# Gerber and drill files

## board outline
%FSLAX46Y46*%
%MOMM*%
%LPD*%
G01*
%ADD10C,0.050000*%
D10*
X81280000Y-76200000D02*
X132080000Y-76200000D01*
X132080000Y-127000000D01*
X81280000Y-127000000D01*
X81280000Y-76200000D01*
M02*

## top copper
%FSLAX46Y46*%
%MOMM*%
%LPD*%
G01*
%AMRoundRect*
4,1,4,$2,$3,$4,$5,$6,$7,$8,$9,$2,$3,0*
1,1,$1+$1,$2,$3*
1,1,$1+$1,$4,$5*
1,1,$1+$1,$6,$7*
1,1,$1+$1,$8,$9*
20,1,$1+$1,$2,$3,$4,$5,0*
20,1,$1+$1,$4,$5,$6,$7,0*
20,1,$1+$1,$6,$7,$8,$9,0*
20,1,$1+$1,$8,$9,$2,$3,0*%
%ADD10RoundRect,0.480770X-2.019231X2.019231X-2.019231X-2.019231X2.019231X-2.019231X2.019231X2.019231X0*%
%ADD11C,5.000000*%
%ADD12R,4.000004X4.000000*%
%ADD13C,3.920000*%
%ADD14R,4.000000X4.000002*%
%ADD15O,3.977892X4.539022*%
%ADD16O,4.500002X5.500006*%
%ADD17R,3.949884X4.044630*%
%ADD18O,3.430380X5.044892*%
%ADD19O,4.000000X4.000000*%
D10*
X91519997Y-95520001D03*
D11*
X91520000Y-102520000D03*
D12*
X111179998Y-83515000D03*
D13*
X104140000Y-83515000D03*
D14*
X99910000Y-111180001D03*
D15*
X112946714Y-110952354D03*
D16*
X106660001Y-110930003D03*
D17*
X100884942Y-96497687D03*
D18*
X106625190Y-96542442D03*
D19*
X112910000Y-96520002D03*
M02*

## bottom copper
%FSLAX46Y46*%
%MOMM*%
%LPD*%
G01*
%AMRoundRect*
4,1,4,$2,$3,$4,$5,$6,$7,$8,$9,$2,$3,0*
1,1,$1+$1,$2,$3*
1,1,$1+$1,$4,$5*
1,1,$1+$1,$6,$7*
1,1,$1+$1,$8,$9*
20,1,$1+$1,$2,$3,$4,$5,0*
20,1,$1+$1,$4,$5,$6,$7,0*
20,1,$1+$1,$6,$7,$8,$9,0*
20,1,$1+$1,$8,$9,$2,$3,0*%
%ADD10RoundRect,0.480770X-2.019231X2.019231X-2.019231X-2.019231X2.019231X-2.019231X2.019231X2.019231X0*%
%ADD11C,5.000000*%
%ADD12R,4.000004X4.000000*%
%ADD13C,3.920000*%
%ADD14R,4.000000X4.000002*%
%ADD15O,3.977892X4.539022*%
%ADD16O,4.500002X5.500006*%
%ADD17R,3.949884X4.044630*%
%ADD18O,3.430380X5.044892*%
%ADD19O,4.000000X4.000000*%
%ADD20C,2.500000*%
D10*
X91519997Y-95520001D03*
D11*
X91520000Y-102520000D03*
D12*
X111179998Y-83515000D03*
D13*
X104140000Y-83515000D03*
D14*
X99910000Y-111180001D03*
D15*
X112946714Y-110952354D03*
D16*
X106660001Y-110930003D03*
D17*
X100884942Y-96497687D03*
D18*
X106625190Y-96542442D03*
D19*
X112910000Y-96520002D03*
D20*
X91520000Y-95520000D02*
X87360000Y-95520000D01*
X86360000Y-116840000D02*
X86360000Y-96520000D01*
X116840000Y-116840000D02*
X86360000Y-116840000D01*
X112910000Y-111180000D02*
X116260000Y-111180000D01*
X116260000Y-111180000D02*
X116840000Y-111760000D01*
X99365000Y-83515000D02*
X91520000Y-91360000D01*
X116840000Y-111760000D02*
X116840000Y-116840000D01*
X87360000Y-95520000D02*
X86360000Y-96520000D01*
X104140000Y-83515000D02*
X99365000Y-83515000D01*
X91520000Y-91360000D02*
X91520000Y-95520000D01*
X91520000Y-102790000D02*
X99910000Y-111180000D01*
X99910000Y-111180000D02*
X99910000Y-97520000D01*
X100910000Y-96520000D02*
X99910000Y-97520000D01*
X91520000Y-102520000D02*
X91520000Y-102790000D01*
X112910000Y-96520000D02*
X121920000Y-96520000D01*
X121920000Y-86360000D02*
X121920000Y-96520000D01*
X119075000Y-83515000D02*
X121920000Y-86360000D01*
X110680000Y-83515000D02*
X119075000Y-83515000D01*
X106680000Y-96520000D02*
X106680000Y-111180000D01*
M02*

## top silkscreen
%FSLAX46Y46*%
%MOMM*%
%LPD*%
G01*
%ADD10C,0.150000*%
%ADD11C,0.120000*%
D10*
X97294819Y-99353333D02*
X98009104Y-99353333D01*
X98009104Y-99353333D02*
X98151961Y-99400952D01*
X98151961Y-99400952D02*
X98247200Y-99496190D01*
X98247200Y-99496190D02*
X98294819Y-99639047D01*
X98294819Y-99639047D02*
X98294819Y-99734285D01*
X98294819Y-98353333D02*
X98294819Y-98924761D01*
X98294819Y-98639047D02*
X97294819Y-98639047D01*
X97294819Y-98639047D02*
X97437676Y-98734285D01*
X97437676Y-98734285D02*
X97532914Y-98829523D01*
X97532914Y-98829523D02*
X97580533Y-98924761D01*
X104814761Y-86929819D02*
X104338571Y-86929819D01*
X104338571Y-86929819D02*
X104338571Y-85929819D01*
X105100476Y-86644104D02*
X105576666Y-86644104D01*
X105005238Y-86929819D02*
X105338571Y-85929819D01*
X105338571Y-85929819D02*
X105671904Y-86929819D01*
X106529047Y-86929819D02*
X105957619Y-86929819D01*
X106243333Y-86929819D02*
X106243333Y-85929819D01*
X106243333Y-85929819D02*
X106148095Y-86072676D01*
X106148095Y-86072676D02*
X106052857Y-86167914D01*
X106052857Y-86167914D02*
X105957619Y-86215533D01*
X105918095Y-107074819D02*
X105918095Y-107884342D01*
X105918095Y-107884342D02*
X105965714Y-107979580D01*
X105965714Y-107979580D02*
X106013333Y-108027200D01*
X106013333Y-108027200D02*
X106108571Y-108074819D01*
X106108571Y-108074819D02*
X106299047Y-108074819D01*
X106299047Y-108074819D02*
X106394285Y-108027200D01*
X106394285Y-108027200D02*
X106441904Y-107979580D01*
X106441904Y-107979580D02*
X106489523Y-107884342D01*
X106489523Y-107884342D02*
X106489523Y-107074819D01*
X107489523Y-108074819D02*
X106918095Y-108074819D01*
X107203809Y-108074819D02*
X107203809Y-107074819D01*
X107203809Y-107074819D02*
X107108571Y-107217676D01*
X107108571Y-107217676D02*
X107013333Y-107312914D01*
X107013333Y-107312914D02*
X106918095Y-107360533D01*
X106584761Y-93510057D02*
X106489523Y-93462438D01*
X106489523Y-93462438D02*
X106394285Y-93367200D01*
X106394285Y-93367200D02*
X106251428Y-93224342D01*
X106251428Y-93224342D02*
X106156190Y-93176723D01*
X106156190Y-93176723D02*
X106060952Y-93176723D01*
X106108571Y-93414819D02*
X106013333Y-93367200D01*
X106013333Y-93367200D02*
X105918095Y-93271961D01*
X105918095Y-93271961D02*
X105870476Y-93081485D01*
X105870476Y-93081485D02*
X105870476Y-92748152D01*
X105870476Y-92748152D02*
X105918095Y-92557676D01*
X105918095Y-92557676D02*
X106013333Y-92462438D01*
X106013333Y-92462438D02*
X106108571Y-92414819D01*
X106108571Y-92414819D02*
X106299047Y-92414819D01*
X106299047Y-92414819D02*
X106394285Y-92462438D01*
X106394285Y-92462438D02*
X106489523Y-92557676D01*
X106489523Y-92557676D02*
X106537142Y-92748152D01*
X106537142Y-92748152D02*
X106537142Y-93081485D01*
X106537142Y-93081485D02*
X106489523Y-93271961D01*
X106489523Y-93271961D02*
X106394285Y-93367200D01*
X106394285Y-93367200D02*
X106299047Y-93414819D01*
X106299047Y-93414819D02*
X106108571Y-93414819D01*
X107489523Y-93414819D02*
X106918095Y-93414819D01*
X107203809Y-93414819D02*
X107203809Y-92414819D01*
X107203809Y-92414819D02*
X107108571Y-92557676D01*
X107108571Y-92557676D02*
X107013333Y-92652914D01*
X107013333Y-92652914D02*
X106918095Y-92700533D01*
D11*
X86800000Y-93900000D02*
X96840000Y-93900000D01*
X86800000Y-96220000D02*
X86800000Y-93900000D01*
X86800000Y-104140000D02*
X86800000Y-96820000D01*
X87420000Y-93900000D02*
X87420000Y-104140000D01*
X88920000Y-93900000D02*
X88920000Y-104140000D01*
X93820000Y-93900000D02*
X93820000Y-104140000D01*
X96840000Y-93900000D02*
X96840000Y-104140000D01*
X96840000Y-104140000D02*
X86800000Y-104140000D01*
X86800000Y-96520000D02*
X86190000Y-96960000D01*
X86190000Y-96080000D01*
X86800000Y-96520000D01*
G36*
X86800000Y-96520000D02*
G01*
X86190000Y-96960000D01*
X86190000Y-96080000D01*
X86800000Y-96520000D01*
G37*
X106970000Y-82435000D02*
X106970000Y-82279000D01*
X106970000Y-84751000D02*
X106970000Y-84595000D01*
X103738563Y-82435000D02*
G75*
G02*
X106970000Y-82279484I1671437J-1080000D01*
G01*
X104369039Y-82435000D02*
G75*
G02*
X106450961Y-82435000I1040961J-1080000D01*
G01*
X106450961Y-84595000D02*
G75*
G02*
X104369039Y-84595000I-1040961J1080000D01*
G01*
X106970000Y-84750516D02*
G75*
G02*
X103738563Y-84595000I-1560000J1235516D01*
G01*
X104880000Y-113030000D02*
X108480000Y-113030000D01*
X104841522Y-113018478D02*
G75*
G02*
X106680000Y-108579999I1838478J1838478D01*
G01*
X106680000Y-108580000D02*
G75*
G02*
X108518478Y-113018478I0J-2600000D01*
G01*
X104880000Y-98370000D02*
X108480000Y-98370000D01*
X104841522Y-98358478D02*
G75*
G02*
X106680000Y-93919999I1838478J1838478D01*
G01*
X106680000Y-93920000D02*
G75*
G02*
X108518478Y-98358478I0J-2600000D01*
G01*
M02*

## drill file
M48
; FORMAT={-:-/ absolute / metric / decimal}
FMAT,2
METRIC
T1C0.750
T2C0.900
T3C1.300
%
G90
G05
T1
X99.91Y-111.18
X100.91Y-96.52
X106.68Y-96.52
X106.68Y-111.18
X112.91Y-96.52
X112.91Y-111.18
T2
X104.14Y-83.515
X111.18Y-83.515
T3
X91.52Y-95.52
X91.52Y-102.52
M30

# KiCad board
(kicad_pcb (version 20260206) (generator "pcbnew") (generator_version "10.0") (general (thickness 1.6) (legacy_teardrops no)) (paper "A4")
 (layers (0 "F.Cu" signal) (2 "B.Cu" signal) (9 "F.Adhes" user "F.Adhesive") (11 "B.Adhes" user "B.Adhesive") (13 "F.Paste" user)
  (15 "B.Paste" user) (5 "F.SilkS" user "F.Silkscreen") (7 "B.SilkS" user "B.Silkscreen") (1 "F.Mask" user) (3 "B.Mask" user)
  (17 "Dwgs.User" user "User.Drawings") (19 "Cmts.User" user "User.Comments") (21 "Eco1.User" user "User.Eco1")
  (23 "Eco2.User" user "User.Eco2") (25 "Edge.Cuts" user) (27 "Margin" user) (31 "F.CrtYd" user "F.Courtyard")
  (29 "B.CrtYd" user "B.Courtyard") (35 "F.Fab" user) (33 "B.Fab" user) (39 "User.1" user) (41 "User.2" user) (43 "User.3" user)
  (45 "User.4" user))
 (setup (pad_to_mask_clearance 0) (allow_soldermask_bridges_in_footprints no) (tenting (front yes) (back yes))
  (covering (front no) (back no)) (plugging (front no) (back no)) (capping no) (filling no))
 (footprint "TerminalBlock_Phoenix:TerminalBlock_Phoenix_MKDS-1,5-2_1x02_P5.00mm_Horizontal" (layer "F.Cu") (at 91.52 96.52 -90)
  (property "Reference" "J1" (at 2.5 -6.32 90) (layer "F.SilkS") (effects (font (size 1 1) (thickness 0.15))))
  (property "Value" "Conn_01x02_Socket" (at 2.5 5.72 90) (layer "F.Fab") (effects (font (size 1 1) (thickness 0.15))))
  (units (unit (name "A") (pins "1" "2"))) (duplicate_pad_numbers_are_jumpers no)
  (fp_line (start -2.62 4.72) (end -2.62 -5.32) (stroke (width 0.12) (type solid)) (layer "F.SilkS"))
  (fp_line (start -0.3 4.72) (end -2.62 4.72) (stroke (width 0.12) (type solid)) (layer "F.SilkS"))
  (fp_line (start 7.62 4.72) (end 0.3 4.72) (stroke (width 0.12) (type solid)) (layer "F.SilkS"))
  (fp_line (start -2.62 4.1) (end 7.62 4.1) (stroke (width 0.12) (type solid)) (layer "F.SilkS"))
  (fp_line (start -2.62 2.6) (end 7.62 2.6) (stroke (width 0.12) (type solid)) (layer "F.SilkS"))
  (fp_line (start -2.62 -2.3) (end 7.62 -2.3) (stroke (width 0.12) (type solid)) (layer "F.SilkS"))
  (fp_line (start -2.62 -5.32) (end 7.62 -5.32) (stroke (width 0.12) (type solid)) (layer "F.SilkS"))
  (fp_line (start 7.62 -5.32) (end 7.62 4.72) (stroke (width 0.12) (type solid)) (layer "F.SilkS"))
  (fp_poly (pts (xy 0 4.72) (xy 0.44 5.33) (xy -0.44 5.33)) (stroke (width 0.12) (type solid)) (fill yes) (layer "F.SilkS"))
  (pad "1" thru_hole roundrect (at -1 0 270) (size 5.000002 5.000002) (drill 1.3 (offset 0.000001 0.000003)) (layers "*.Cu" "*.Mask")
   (remove_unused_layers no) (roundrect_rratio 0.096154) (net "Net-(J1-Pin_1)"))
  (pad "2" thru_hole circle (at 6 0 270) (size 5 5) (drill 1.3) (layers "*.Cu" "*.Mask") (remove_unused_layers no) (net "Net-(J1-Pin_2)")))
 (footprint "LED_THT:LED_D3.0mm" (layer "F.Cu") (at 106.68 83.515 180)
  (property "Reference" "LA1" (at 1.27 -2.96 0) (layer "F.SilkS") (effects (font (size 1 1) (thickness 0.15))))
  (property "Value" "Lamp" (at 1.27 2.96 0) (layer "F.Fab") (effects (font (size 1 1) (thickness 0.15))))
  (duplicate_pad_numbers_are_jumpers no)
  (fp_line (start -0.29 1.08) (end -0.29 1.236) (stroke (width 0.12) (type solid)) (layer "F.SilkS"))
  (fp_line (start -0.29 -1.236) (end -0.29 -1.08) (stroke (width 0.12) (type solid)) (layer "F.SilkS"))
  (fp_arc (start 2.941437 1.08) (mid 1.36566 1.987699) (end -0.29 1.235516) (stroke (width 0.12) (type solid)) (layer "F.SilkS"))
  (fp_arc (start 2.310961 1.08) (mid 1.27 1.5) (end 0.229039 1.08) (stroke (width 0.12) (type solid)) (layer "F.SilkS"))
  (fp_arc (start 0.229039 -1.08) (mid 1.27 -1.5) (end 2.310961 -1.08) (stroke (width 0.12) (type solid)) (layer "F.SilkS"))
  (fp_arc (start -0.29 -1.235516) (mid 1.36566 -1.987699) (end 2.941437 -1.08) (stroke (width 0.12) (type solid)) (layer "F.SilkS"))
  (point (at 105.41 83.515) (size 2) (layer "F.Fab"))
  (pad "1" thru_hole rect (at -4.5 0 180) (size 4.000004 4) (drill 0.9 (offset 0.000002 0)) (layers "*.Cu" "*.Mask")
   (remove_unused_layers no) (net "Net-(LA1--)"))
  (pad "2" thru_hole circle (at 2.54 0 180) (size 3.92 3.92) (drill 0.9) (layers "*.Cu" "*.Mask") (remove_unused_layers no)
   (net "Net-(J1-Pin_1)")))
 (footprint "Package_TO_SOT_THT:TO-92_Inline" (layer "F.Cu") (at 105.41 111.18)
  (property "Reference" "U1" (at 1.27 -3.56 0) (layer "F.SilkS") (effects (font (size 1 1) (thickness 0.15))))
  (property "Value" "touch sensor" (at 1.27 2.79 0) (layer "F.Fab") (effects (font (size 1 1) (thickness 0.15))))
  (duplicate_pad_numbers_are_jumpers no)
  (fp_line (start -0.53 1.85) (end 3.07 1.85) (stroke (width 0.12) (type solid)) (layer "F.SilkS"))
  (fp_arc (start -0.568478 1.838478) (mid -1.132087 -0.994977) (end 1.27 -2.6) (stroke (width 0.12) (type solid)) (layer "F.SilkS"))
  (fp_arc (start 1.27 -2.6) (mid 3.672087 -0.994977) (end 3.108478 1.838478) (stroke (width 0.12) (type solid)) (layer "F.SilkS"))
  (pad "1" thru_hole rect (at -5.5 0) (size 4 4.000002) (drill 0.75 (offset 0 0.000001)) (layers "*.Cu" "*.Mask") (remove_unused_layers no)
   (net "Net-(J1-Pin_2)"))
  (pad "2" thru_hole oval (at 7.5 0) (size 3.977892 4.539022) (drill 0.75 (offset 0.036714 -0.227646)) (layers "*.Cu" "*.Mask")
   (remove_unused_layers no) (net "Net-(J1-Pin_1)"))
  (pad "3" thru_hole oval (at 1.27 0) (size 4.500002 5.500006) (drill 0.75 (offset -0.019999 -0.249997)) (layers "*.Cu" "*.Mask")
   (remove_unused_layers no) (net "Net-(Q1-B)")))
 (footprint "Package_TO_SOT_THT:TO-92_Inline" (layer "F.Cu") (at 105.41 96.52)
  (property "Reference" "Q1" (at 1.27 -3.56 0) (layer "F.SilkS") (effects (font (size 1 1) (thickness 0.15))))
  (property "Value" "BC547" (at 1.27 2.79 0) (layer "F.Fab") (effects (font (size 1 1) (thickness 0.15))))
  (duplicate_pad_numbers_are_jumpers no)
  (fp_line (start -0.53 1.85) (end 3.07 1.85) (stroke (width 0.12) (type solid)) (layer "F.SilkS"))
  (fp_arc (start -0.568478 1.838478) (mid -1.132087 -0.994977) (end 1.27 -2.6) (stroke (width 0.12) (type solid)) (layer "F.SilkS"))
  (fp_arc (start 1.27 -2.6) (mid 3.672087 -0.994977) (end 3.108478 1.838478) (stroke (width 0.12) (type solid)) (layer "F.SilkS"))
  (pad "1" thru_hole rect (at -4.5 0) (size 3.949884 4.04463) (drill 0.75 (offset -0.025058 -0.022313)) (layers "*.Cu" "*.Mask")
   (remove_unused_layers no) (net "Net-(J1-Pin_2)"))
  (pad "2" thru_hole oval (at 1.27 0) (size 3.43038 5.044892) (drill 0.75 (offset -0.05481 0.022442)) (layers "*.Cu" "*.Mask")
   (remove_unused_layers no) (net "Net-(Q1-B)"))
  (pad "3" thru_hole oval (at 7.5 0) (size 4 4) (drill 0.75 (offset 0 0.000002)) (layers "*.Cu" "*.Mask") (remove_unused_layers no)
   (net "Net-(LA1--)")))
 (gr_rect (start 81.28 76.2) (end 132.08 127) (stroke (width 0.05) (type default)) (fill no) (layer "Edge.Cuts"))
 (segment (start 91.52 95.52) (end 87.36 95.52) (width 2.5) (layer "B.Cu") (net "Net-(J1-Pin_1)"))
 (segment (start 86.36 116.84) (end 86.36 96.52) (width 2.5) (layer "B.Cu") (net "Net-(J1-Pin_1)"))
 (segment (start 116.84 116.84) (end 86.36 116.84) (width 2.5) (layer "B.Cu") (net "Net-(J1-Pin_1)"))
 (segment (start 112.91 111.18) (end 116.26 111.18) (width 2.5) (layer "B.Cu") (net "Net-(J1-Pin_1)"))
 (segment (start 116.26 111.18) (end 116.84 111.76) (width 2.5) (layer "B.Cu") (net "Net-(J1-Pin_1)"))
 (segment (start 99.365 83.515) (end 91.52 91.36) (width 2.5) (layer "B.Cu") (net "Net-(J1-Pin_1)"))
 (segment (start 116.84 111.76) (end 116.84 116.84) (width 2.5) (layer "B.Cu") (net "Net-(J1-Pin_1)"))
 (segment (start 87.36 95.52) (end 86.36 96.52) (width 2.5) (layer "B.Cu") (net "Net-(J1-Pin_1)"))
 (segment (start 104.14 83.515) (end 99.365 83.515) (width 2.5) (layer "B.Cu") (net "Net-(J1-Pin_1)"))
 (segment (start 91.52 91.36) (end 91.52 95.52) (width 2.5) (layer "B.Cu") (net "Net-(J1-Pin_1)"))
 (segment (start 91.52 102.79) (end 99.91 111.18) (width 2.5) (layer "B.Cu") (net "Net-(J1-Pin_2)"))
 (segment (start 99.91 111.18) (end 99.91 97.52) (width 2.5) (layer "B.Cu") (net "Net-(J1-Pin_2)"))
 (segment (start 100.91 96.52) (end 99.91 97.52) (width 2.5) (layer "B.Cu") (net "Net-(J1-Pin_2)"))
 (segment (start 91.52 102.52) (end 91.52 102.79) (width 2.5) (layer "B.Cu") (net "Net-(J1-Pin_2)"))
 (segment (start 112.91 96.52) (end 121.92 96.52) (width 2.5) (layer "B.Cu") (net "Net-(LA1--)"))
 (segment (start 121.92 86.36) (end 121.92 96.52) (width 2.5) (layer "B.Cu") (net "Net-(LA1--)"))
 (segment (start 119.075 83.515) (end 121.92 86.36) (width 2.5) (layer "B.Cu") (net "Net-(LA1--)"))
 (segment (start 110.68 83.515) (end 119.075 83.515) (width 2.5) (layer "B.Cu") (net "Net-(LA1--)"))
 (segment (start 106.68 96.52) (end 106.68 111.18) (width 2.5) (layer "B.Cu") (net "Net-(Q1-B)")))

